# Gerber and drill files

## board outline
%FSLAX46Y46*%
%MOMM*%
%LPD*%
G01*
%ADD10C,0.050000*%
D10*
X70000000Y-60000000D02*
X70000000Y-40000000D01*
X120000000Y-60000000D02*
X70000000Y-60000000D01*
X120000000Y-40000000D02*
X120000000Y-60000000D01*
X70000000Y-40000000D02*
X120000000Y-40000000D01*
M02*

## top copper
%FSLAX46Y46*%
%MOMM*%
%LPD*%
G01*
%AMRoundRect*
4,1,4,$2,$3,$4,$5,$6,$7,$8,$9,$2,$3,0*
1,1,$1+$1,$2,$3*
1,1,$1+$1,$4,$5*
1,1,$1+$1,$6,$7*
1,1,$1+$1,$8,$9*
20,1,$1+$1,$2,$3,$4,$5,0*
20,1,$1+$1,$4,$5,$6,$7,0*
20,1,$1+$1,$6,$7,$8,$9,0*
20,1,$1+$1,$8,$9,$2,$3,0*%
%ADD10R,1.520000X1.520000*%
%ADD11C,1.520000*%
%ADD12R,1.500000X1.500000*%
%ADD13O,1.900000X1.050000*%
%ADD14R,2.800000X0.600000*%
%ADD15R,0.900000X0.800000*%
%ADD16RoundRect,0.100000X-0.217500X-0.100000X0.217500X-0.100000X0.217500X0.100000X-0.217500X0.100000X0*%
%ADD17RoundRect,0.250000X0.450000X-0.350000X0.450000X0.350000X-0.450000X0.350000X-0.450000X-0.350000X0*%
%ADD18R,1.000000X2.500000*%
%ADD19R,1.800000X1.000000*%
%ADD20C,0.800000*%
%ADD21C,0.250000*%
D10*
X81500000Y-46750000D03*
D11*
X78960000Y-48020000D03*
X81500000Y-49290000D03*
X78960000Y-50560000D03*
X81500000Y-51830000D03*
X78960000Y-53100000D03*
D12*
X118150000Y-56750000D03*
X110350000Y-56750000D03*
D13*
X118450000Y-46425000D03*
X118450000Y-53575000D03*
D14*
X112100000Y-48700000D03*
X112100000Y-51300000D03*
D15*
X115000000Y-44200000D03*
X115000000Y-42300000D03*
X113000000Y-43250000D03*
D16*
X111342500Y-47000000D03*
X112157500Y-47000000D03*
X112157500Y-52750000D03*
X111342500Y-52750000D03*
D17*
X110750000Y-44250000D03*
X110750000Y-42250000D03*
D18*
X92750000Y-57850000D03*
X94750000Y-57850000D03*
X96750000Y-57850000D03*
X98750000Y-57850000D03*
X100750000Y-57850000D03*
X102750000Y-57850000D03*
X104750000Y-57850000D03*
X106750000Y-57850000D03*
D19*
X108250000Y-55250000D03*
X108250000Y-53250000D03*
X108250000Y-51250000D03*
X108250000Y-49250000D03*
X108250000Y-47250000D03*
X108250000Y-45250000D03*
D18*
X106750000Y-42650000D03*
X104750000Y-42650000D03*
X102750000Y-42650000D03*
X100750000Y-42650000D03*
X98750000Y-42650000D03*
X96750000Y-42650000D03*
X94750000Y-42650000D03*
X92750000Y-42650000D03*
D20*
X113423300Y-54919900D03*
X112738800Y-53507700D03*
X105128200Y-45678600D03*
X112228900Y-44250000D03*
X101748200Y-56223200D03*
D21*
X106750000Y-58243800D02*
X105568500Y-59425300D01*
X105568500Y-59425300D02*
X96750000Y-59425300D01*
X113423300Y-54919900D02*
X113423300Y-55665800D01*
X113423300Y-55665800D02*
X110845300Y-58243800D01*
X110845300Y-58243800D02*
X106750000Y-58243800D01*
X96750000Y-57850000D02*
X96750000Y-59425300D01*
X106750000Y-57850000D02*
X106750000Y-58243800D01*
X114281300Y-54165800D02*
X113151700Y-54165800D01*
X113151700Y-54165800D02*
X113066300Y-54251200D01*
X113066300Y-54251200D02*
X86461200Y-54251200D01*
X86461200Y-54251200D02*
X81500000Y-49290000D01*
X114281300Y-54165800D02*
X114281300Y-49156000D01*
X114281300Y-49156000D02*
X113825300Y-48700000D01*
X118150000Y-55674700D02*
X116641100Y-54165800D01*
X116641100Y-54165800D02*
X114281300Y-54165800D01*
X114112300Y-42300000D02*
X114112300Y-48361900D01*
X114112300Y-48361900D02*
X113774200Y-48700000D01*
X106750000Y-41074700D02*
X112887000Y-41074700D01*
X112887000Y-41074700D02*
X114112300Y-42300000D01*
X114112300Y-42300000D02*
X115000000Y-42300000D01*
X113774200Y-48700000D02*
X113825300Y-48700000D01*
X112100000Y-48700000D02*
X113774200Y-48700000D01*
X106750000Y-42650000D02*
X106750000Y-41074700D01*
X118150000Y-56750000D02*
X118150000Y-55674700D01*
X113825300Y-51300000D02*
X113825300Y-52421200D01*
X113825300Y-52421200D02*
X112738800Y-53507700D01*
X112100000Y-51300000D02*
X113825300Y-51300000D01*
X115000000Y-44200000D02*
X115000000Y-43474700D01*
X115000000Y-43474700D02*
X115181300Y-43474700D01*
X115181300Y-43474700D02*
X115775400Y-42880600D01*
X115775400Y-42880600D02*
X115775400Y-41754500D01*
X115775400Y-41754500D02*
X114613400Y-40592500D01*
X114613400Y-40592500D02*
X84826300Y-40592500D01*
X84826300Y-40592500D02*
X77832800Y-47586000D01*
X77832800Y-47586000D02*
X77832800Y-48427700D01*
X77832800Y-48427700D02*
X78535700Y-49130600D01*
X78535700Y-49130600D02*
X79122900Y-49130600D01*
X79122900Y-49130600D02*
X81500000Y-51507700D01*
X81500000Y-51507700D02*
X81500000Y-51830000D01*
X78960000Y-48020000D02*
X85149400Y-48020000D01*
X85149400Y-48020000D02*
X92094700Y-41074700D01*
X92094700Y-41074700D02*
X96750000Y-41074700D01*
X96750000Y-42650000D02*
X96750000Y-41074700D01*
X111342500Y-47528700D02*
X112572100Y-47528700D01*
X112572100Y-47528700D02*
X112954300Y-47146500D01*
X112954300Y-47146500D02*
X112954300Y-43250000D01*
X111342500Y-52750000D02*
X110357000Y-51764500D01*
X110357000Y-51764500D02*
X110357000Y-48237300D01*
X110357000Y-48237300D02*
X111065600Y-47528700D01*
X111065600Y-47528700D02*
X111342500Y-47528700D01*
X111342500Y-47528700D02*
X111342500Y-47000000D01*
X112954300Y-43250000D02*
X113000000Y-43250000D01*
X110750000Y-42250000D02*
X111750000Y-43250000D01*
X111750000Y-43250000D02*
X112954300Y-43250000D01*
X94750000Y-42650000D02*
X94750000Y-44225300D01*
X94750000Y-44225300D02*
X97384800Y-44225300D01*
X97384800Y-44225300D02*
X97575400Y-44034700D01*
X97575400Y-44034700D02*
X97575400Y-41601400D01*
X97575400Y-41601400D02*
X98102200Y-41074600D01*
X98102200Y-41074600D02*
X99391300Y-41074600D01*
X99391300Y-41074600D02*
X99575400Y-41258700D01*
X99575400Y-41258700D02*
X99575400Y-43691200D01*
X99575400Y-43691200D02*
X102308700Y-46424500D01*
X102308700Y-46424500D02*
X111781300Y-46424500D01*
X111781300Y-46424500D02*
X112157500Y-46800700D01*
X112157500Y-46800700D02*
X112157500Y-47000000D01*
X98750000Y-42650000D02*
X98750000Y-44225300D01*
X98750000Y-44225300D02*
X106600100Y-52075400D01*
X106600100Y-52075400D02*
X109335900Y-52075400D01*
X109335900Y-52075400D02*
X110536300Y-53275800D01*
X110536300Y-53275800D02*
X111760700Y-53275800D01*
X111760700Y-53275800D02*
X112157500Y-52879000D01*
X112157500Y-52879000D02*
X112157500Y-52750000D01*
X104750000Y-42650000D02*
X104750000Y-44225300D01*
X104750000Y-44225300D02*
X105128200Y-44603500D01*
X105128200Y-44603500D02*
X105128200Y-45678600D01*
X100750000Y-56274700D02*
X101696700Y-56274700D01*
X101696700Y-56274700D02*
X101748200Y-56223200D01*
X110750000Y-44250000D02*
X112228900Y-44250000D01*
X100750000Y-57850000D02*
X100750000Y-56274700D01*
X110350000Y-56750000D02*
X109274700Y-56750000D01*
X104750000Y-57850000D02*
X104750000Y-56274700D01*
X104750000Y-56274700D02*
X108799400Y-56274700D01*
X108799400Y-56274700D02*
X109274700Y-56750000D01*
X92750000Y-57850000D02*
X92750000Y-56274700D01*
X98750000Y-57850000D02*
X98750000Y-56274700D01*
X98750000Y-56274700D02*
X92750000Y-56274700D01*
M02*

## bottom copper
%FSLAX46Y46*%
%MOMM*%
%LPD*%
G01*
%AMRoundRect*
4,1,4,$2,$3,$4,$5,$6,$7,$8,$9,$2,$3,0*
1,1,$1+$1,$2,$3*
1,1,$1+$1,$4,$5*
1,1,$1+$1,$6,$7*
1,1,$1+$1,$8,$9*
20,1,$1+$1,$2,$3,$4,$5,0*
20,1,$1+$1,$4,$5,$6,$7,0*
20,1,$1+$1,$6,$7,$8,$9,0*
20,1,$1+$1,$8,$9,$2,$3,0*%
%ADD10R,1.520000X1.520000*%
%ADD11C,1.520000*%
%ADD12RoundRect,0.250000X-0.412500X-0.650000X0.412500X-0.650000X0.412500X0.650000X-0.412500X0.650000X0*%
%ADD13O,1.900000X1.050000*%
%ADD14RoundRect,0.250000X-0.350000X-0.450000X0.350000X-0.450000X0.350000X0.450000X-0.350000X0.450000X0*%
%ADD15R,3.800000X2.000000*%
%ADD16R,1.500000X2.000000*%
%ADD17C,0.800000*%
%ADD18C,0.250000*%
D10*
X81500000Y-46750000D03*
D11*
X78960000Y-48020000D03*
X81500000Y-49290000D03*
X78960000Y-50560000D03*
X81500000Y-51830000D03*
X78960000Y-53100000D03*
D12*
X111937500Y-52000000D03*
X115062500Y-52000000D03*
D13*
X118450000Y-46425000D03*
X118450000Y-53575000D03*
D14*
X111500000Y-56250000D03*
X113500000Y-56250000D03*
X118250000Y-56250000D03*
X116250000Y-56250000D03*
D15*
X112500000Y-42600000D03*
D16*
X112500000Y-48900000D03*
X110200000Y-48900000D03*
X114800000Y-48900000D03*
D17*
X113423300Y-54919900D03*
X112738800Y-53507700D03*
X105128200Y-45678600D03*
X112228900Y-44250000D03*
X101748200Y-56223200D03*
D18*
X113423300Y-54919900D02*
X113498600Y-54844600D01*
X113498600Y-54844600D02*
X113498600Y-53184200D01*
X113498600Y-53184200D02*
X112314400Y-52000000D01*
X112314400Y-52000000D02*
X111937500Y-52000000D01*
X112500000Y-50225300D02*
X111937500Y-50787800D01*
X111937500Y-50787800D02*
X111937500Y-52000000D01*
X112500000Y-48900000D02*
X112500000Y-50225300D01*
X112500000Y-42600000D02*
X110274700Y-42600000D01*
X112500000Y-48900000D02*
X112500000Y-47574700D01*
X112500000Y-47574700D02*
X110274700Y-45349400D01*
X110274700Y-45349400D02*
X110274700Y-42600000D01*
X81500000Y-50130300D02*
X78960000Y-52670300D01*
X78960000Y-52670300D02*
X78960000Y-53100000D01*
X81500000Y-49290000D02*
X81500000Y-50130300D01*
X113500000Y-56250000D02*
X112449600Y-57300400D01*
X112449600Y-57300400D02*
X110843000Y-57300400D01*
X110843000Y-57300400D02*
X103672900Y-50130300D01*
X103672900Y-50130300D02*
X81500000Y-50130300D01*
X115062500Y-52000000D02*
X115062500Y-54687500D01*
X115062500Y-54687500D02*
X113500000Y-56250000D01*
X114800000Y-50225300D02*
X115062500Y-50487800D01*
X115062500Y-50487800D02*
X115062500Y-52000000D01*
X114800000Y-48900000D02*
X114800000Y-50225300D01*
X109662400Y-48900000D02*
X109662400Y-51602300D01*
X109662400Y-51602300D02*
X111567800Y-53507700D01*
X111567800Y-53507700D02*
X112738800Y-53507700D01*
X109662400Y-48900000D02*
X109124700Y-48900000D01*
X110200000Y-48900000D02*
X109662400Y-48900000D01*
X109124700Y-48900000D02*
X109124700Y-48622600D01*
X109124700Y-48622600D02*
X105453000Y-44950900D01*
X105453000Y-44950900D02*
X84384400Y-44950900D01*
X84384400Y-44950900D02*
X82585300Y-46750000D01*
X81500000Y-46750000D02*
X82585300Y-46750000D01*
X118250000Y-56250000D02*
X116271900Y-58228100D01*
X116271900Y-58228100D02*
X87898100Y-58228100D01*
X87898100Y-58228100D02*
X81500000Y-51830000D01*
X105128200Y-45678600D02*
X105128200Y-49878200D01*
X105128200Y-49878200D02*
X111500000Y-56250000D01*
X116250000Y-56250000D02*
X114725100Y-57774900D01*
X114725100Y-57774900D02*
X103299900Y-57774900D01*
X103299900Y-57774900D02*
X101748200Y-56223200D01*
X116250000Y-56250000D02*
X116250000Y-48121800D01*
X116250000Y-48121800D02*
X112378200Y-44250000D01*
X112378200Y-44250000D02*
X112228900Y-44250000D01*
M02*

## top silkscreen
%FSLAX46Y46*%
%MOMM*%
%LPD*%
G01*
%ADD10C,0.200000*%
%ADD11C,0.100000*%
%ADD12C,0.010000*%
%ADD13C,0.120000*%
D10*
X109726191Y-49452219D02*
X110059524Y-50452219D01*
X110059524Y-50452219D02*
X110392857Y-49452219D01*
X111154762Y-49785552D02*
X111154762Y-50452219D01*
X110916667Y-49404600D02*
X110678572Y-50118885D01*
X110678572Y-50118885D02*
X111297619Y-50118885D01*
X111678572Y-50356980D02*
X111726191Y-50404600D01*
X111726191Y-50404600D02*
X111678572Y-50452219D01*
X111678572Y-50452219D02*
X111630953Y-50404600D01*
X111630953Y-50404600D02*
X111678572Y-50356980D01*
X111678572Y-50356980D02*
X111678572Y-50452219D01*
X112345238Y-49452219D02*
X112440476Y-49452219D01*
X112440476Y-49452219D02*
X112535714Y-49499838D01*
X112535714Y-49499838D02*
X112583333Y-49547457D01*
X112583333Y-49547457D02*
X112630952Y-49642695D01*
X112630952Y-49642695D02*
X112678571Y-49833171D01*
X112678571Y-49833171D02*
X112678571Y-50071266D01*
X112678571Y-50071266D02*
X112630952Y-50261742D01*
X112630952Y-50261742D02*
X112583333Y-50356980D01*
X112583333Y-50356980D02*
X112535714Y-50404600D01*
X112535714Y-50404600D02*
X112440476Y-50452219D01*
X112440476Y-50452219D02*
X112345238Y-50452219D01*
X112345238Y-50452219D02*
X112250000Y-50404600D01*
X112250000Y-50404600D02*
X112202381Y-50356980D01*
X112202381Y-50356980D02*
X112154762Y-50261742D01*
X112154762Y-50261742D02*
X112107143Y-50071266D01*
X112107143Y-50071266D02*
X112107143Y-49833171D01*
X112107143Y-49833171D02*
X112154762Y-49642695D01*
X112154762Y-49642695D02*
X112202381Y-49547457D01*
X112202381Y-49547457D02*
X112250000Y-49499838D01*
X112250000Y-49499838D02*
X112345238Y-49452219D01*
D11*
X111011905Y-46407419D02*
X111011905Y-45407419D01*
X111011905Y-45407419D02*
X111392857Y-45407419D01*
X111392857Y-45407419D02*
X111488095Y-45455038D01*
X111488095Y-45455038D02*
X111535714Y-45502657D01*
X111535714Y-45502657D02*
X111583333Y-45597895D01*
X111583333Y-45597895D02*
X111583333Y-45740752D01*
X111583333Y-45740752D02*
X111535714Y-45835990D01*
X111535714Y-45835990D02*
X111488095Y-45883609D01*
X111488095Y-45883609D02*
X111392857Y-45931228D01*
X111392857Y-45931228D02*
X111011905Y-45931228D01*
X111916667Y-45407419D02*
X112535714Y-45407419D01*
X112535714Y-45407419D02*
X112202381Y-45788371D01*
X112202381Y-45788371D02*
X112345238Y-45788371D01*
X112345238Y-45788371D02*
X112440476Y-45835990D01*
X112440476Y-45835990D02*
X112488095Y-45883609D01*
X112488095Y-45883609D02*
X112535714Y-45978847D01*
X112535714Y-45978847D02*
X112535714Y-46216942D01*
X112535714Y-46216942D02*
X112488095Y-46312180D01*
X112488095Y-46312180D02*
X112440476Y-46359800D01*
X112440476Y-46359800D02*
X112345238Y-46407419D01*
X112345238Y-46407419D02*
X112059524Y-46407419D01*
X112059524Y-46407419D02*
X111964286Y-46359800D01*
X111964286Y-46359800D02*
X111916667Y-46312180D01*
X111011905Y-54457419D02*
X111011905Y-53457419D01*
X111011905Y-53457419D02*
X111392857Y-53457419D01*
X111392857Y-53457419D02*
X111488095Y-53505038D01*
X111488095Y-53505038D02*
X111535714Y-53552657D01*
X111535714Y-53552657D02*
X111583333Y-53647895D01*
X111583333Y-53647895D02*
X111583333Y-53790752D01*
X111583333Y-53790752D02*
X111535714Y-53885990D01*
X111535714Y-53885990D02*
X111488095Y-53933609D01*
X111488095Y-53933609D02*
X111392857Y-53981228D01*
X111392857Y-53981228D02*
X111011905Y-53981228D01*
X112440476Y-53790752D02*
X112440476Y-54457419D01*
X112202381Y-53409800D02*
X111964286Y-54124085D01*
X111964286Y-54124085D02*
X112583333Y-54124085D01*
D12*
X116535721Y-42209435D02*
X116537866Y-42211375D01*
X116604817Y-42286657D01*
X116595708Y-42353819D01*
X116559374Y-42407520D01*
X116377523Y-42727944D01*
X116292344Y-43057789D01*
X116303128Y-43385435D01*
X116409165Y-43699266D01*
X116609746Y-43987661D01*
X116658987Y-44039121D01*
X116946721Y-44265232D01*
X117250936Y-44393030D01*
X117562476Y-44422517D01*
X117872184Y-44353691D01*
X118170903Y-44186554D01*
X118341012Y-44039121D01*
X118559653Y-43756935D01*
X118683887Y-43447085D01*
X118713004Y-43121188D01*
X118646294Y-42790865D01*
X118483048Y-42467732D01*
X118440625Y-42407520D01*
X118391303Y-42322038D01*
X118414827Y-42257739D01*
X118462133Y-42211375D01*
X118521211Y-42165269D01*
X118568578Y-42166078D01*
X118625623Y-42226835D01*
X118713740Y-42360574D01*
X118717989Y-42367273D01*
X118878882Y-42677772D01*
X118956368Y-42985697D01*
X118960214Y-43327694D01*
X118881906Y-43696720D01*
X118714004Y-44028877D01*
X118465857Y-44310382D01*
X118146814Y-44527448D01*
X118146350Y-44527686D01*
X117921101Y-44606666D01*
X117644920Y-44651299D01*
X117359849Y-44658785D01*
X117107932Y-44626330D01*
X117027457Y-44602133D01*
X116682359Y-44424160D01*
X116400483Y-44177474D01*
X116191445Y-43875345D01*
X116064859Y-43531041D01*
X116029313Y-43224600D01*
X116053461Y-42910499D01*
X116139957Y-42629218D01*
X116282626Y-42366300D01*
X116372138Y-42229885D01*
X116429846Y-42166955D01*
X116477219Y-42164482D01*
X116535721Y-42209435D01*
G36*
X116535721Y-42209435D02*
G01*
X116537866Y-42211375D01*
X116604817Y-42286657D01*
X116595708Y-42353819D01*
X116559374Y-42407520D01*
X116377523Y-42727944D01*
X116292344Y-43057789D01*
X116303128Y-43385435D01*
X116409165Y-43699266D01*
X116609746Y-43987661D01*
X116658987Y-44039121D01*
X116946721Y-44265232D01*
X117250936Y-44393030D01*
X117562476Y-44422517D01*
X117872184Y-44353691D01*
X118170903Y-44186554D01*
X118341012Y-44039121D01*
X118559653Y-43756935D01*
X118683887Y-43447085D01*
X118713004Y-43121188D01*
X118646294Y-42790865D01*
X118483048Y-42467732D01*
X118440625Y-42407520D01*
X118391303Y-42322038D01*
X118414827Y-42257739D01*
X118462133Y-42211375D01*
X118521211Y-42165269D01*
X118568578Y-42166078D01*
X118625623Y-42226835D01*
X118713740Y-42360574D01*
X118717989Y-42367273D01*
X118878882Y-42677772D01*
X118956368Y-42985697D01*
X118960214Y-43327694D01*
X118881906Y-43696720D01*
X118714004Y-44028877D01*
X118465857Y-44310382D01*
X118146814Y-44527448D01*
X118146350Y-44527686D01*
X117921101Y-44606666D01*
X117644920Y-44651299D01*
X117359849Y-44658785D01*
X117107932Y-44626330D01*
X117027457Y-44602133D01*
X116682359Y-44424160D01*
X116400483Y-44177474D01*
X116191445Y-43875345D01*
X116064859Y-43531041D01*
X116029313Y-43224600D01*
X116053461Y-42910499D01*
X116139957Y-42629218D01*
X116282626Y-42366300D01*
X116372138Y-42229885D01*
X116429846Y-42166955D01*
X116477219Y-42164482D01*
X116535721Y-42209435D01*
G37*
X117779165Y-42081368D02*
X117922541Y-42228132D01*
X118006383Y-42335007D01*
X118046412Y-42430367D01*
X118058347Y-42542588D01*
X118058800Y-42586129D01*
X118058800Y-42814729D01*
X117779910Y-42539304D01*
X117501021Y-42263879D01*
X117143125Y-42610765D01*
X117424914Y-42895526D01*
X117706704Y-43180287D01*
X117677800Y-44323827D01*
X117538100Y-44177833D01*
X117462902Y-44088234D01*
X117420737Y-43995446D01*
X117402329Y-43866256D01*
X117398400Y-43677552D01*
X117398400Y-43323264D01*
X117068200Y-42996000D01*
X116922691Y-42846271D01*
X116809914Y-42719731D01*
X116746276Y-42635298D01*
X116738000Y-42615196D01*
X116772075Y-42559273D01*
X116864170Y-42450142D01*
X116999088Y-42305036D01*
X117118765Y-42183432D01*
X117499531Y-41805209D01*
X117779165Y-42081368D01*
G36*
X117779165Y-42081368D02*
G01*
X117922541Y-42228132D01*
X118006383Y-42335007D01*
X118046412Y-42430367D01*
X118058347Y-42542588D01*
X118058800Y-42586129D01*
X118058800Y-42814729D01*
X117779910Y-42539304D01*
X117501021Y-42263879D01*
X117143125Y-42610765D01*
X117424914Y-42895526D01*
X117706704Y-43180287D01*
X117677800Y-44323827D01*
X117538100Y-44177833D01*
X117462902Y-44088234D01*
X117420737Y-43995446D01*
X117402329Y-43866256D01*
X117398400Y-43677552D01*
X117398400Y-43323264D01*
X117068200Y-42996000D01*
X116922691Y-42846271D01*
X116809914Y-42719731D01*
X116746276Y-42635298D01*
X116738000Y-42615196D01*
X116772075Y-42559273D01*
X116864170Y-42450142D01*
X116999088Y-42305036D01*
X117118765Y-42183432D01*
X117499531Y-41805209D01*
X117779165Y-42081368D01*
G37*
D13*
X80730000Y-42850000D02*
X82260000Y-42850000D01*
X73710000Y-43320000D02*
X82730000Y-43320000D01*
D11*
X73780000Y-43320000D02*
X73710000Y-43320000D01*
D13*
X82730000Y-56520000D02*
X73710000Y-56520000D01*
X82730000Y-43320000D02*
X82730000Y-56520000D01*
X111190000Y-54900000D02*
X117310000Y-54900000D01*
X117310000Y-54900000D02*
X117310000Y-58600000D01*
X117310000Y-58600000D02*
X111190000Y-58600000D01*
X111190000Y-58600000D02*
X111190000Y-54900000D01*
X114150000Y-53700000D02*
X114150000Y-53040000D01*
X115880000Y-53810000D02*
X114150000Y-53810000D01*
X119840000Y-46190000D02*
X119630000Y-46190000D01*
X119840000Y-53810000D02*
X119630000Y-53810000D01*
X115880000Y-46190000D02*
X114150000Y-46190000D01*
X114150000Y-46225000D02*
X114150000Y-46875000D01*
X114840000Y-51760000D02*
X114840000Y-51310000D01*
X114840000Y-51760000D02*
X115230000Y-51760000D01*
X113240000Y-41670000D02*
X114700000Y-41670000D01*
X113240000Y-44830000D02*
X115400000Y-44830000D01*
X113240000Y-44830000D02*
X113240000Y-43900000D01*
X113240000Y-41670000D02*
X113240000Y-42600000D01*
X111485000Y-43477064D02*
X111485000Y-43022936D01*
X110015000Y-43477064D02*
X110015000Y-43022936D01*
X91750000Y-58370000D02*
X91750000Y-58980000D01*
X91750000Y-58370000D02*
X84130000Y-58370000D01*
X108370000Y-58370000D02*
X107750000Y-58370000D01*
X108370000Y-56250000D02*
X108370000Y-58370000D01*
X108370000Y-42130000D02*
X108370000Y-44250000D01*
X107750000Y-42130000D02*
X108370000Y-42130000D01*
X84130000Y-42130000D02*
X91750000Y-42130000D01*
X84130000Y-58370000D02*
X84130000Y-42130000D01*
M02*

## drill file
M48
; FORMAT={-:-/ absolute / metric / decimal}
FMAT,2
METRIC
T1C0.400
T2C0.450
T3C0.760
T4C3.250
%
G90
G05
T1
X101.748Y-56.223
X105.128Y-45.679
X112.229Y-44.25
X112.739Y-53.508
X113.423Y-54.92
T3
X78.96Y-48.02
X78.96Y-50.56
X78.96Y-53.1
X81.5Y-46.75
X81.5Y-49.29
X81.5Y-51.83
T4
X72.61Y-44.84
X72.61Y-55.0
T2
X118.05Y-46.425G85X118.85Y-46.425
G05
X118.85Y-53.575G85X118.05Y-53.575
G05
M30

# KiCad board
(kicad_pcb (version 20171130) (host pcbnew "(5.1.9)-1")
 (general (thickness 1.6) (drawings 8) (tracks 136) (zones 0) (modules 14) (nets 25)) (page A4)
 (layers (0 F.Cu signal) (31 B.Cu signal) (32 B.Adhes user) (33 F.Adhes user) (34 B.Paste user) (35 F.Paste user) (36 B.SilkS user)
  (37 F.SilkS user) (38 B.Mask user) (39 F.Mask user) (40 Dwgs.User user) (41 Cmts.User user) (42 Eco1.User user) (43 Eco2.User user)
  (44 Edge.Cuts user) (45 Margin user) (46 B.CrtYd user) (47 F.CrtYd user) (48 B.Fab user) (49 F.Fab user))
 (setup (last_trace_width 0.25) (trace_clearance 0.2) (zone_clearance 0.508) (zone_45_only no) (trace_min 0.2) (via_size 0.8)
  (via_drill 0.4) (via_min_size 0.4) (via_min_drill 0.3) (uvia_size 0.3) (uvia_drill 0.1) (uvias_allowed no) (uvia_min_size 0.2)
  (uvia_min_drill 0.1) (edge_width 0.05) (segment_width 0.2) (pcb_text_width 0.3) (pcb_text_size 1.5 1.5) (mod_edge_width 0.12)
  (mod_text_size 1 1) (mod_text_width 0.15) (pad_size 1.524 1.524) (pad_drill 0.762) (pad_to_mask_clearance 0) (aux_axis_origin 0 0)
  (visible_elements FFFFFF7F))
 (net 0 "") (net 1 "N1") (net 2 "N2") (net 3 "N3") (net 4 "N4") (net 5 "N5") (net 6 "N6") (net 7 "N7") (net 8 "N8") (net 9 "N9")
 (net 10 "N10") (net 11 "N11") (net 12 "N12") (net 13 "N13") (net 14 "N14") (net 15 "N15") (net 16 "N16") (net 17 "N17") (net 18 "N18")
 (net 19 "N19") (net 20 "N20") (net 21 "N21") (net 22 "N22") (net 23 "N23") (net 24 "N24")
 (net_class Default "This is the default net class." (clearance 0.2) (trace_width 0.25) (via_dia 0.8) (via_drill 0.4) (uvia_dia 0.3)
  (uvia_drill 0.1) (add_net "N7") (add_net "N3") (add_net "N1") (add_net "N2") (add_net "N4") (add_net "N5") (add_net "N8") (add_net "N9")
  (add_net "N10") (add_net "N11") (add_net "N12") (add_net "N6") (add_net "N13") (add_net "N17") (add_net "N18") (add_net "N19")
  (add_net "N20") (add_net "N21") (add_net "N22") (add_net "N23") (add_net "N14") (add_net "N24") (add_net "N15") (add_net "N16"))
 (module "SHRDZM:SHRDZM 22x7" (layer B.Cu) (at 96.25 49 180)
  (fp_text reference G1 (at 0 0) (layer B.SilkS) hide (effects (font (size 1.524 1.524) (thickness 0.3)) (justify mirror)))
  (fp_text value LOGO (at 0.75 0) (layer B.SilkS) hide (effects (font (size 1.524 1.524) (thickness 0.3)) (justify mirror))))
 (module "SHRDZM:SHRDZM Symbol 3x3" (layer F.Cu) (at 117.5 43.25)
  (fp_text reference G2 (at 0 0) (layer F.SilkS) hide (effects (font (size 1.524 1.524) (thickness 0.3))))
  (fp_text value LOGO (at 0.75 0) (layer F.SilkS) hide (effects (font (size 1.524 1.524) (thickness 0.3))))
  (fp_poly
   (pts (xy -0.964279 -1.040565) (xy -0.962134 -1.038625) (xy -0.895183 -0.963343) (xy -0.904292 -0.896181) (xy -0.940626 -0.84248)
    (xy -1.122477 -0.522056) (xy -1.207656 -0.192211) (xy -1.196872 0.135435) (xy -1.090835 0.449266) (xy -0.890254 0.737661)
    (xy -0.841013 0.789121) (xy -0.553279 1.015232) (xy -0.249064 1.14303) (xy 0.062476 1.172517) (xy 0.372184 1.103691)
    (xy 0.670903 0.936554) (xy 0.841012 0.789121) (xy 1.059653 0.506935) (xy 1.183887 0.197085) (xy 1.213004 -0.128812)
    (xy 1.146294 -0.459135) (xy 0.983048 -0.782268) (xy 0.940625 -0.84248) (xy 0.891303 -0.927962) (xy 0.914827 -0.992261)
    (xy 0.962133 -1.038625) (xy 1.021211 -1.084731) (xy 1.068578 -1.083922) (xy 1.125623 -1.023165) (xy 1.21374 -0.889426)
    (xy 1.217989 -0.882727) (xy 1.378882 -0.572228) (xy 1.456368 -0.264303) (xy 1.460214 0.077694) (xy 1.381906 0.44672)
    (xy 1.214004 0.778877) (xy 0.965857 1.060382) (xy 0.646814 1.277448) (xy 0.64635 1.277686) (xy 0.421101 1.356666) (xy 0.14492 1.401299)
    (xy -0.140151 1.408785) (xy -0.392068 1.37633) (xy -0.472543 1.352133) (xy -0.817641 1.17416) (xy -1.099517 0.927474)
    (xy -1.308555 0.625345) (xy -1.435141 0.281041) (xy -1.470687 -0.0254) (xy -1.446539 -0.339501) (xy -1.360043 -0.620782)
    (xy -1.217374 -0.8837) (xy -1.127862 -1.020115) (xy -1.070154 -1.083045) (xy -1.022781 -1.085518) (xy -0.964279 -1.040565))
   (layer F.SilkS) (width 0.01))
  (fp_poly
   (pts (xy 0.279165 -1.168632) (xy 0.422541 -1.021868) (xy 0.506383 -0.914993) (xy 0.546412 -0.819633) (xy 0.558347 -0.707412)
    (xy 0.5588 -0.663871) (xy 0.5588 -0.435271) (xy 0.27991 -0.710696) (xy 0.001021 -0.986121) (xy -0.356875 -0.639235)
    (xy -0.075086 -0.354474) (xy 0.206704 -0.069713) (xy 0.1778 1.073827) (xy 0.0381 0.927833) (xy -0.037098 0.838234)
    (xy -0.079263 0.745446) (xy -0.097671 0.616256) (xy -0.1016 0.427552) (xy -0.1016 0.073264) (xy -0.4318 -0.254) (xy -0.577309 -0.403729)
    (xy -0.690086 -0.530269) (xy -0.753724 -0.614702) (xy -0.762 -0.634804) (xy -0.727925 -0.690727) (xy -0.63583 -0.799858)
    (xy -0.500912 -0.944964) (xy -0.381235 -1.066568) (xy -0.000469 -1.444791) (xy 0.279165 -1.168632))
   (layer F.SilkS) (width 0.01)))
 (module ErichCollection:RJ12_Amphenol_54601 (layer F.Cu) (at 81.5 46.75 270)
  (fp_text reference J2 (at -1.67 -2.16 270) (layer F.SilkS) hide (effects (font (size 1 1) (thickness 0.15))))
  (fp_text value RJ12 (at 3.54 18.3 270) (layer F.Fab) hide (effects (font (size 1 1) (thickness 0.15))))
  (fp_line (start -3.9 0.77) (end -3.9 -0.76) (layer F.SilkS) (width 0.12))
  (fp_line (start -3.43 7.79) (end -3.43 -1.23) (layer F.SilkS) (width 0.12))
  (fp_line (start -3.43 7.72) (end -3.43 7.79) (layer F.SilkS) (width 0.1))
  (fp_line (start 9.77 -1.23) (end 9.77 7.79) (layer F.SilkS) (width 0.12))
  (fp_line (start -3.43 -1.23) (end 9.77 -1.23) (layer F.SilkS) (width 0.12))
  (pad 1 thru_hole rect (at 0 0 270) (size 1.52 1.52) (drill 0.76) (layers *.Cu *.Mask) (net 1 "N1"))
  (pad "" np_thru_hole circle (at -1.91 8.89 270) (size 3.25 3.25) (drill 3.25) (layers *.Cu *.Mask))
  (pad 2 thru_hole circle (at 1.27 2.54 270) (size 1.52 1.52) (drill 0.76) (layers *.Cu *.Mask) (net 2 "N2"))
  (pad 3 thru_hole circle (at 2.54 0 270) (size 1.52 1.52) (drill 0.76) (layers *.Cu *.Mask) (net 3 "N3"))
  (pad 4 thru_hole circle (at 3.81 2.54 270) (size 1.52 1.52) (drill 0.76) (layers *.Cu *.Mask) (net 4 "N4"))
  (pad 5 thru_hole circle (at 5.08 0 270) (size 1.52 1.52) (drill 0.76) (layers *.Cu *.Mask) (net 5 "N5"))
  (pad 6 thru_hole circle (at 6.35 2.54 270) (size 1.52 1.52) (drill 0.76) (layers *.Cu *.Mask) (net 3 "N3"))
  (pad "" np_thru_hole circle (at 8.25 8.89 270) (size 3.25 3.25) (drill 3.25) (layers *.Cu *.Mask)))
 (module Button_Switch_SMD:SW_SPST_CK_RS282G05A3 (layer F.Cu) (at 114.25 56.75)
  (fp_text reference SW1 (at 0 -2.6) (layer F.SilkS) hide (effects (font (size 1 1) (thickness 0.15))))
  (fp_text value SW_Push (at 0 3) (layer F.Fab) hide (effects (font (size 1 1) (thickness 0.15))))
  (fp_line (start -3.06 -1.85) (end 3.06 -1.85) (layer F.SilkS) (width 0.12))
  (fp_line (start 3.06 -1.85) (end 3.06 1.85) (layer F.SilkS) (width 0.12))
  (fp_line (start 3.06 1.85) (end -3.06 1.85) (layer F.SilkS) (width 0.12))
  (fp_line (start -3.06 1.85) (end -3.06 -1.85) (layer F.SilkS) (width 0.12))
  (pad 2 smd rect (at 3.9 0) (size 1.5 1.5) (layers F.Cu F.Paste F.Mask) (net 3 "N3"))
  (pad 1 smd rect (at -3.9 0) (size 1.5 1.5) (layers F.Cu F.Paste F.Mask) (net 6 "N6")))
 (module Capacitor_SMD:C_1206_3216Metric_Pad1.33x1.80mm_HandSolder (layer B.Cu) (at 113.5 52)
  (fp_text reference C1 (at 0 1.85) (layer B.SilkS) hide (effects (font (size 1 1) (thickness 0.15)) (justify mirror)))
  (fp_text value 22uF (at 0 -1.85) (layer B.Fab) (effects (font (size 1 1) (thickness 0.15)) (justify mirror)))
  (pad 1 smd roundrect (at -1.5625 0) (size 1.325 1.8) (layers B.Cu B.Paste B.Mask) (roundrect_rratio 0.188679) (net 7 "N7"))
  (pad 2 smd roundrect (at 1.5625 0) (size 1.325 1.8) (layers B.Cu B.Paste B.Mask) (roundrect_rratio 0.188679) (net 3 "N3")))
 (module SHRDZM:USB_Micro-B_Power (layer F.Cu) (at 117.25 50 90)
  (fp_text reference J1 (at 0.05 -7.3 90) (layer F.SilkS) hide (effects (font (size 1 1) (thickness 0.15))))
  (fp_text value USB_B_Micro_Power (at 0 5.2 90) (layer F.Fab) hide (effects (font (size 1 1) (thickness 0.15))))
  (fp_line (start -3.7 -3.1) (end -3.04 -3.1) (layer F.SilkS) (width 0.12))
  (fp_line (start -3.81 -1.37) (end -3.81 -3.1) (layer F.SilkS) (width 0.12))
  (fp_line (start 3.81 2.59) (end 3.81 2.38) (layer F.SilkS) (width 0.12))
  (fp_line (start -3.81 2.59) (end -3.81 2.38) (layer F.SilkS) (width 0.12))
  (fp_line (start 3.81 -1.37) (end 3.81 -3.1) (layer F.SilkS) (width 0.12))
  (fp_line (start 3.775 -3.1) (end 3.125 -3.1) (layer F.SilkS) (width 0.12))
  (fp_line (start -1.76 -2.41) (end -1.31 -2.41) (layer F.SilkS) (width 0.12))
  (fp_line (start -1.76 -2.41) (end -1.76 -2.02) (layer F.SilkS) (width 0.12))
  (pad "" thru_hole oval (at 3.575 1.2 90) (size 1.05 1.9) (drill oval 0.45 1.25) (layers *.Cu *.Mask))
  (pad "" thru_hole oval (at -3.575 1.2 270) (size 1.05 1.9) (drill oval 0.45 1.25) (layers *.Cu *.Mask))
  (pad 5 smd rect (at 1.3 -5.15 90) (size 0.6 2.8) (layers F.Cu F.Paste F.Mask) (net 3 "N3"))
  (pad 1 smd rect (at -1.3 -5.15 90) (size 0.6 2.8) (layers F.Cu F.Paste F.Mask) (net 1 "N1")))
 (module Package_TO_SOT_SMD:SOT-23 (layer F.Cu) (at 114 43.25 180)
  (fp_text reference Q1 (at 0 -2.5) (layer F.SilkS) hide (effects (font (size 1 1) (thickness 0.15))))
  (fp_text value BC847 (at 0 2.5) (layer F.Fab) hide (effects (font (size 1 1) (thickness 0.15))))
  (fp_line (start 0.76 1.58) (end -0.7 1.58) (layer F.SilkS) (width 0.12))
  (fp_line (start 0.76 -1.58) (end -1.4 -1.58) (layer F.SilkS) (width 0.12))
  (fp_line (start 0.76 -1.58) (end 0.76 -0.65) (layer F.SilkS) (width 0.12))
  (fp_line (start 0.76 1.58) (end 0.76 0.65) (layer F.SilkS) (width 0.12))
  (pad 1 smd rect (at -1 -0.95 180) (size 0.9 0.8) (layers F.Cu F.Paste F.Mask) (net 5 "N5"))
  (pad 2 smd rect (at -1 0.95 180) (size 0.9 0.8) (layers F.Cu F.Paste F.Mask) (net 3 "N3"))
  (pad 3 smd rect (at 1 0 180) (size 0.9 0.8) (layers F.Cu F.Paste F.Mask) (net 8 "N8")))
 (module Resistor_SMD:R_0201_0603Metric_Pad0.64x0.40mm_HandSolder (layer F.Cu) (at 111.75 47)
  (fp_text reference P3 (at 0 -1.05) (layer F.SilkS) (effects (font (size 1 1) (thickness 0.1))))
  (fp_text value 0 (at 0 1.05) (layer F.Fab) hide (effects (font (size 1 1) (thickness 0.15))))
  (pad "" smd roundrect (at -0.4325 0) (size 0.458 0.36) (layers F.Paste) (roundrect_rratio 0.25))
  (pad "" smd roundrect (at 0.4325 0) (size 0.458 0.36) (layers F.Paste) (roundrect_rratio 0.25))
  (pad 1 smd roundrect (at -0.4075 0) (size 0.635 0.4) (layers F.Cu F.Mask) (roundrect_rratio 0.25) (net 8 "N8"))
  (pad 2 smd roundrect (at 0.4075 0) (size 0.635 0.4) (layers F.Cu F.Mask) (roundrect_rratio 0.25) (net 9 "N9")))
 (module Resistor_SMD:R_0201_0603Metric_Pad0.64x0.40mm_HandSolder (layer F.Cu) (at 111.75 52.75)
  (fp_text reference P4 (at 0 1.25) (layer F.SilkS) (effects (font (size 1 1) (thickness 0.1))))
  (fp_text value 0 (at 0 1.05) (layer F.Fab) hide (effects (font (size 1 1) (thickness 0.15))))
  (pad 2 smd roundrect (at 0.4075 0) (size 0.635 0.4) (layers F.Cu F.Mask) (roundrect_rratio 0.25) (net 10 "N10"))
  (pad 1 smd roundrect (at -0.4075 0) (size 0.635 0.4) (layers F.Cu F.Mask) (roundrect_rratio 0.25) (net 8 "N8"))
  (pad "" smd roundrect (at 0.4325 0) (size 0.458 0.36) (layers F.Paste) (roundrect_rratio 0.25))
  (pad "" smd roundrect (at -0.4325 0) (size 0.458 0.36) (layers F.Paste) (roundrect_rratio 0.25)))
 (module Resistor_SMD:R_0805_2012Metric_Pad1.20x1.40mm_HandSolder (layer B.Cu) (at 112.5 56.25)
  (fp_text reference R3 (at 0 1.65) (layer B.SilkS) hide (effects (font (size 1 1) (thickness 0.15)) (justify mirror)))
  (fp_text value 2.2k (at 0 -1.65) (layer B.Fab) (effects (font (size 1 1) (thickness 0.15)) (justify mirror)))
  (pad 1 smd roundrect (at -1 0) (size 1.2 1.4) (layers B.Cu B.Paste B.Mask) (roundrect_rratio 0.208333) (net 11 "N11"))
  (pad 2 smd roundrect (at 1 0) (size 1.2 1.4) (layers B.Cu B.Paste B.Mask) (roundrect_rratio 0.208333) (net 3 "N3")))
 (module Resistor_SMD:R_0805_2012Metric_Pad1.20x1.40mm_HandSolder (layer F.Cu) (at 110.75 43.25 90)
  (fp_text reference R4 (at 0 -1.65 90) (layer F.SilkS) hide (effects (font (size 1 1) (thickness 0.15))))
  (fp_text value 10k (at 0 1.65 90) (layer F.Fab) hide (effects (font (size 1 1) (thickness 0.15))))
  (fp_line (start -0.227064 0.735) (end 0.227064 0.735) (layer F.SilkS) (width 0.12))
  (fp_line (start -0.227064 -0.735) (end 0.227064 -0.735) (layer F.SilkS) (width 0.12))
  (pad 1 smd roundrect (at -1 0 90) (size 1.2 1.4) (layers F.Cu F.Paste F.Mask) (roundrect_rratio 0.208333) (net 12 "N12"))
  (pad 2 smd roundrect (at 1 0 90) (size 1.2 1.4) (layers F.Cu F.Paste F.Mask) (roundrect_rratio 0.208333) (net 8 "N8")))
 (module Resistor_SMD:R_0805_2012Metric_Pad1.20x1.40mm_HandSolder (layer B.Cu) (at 117.25 56.25)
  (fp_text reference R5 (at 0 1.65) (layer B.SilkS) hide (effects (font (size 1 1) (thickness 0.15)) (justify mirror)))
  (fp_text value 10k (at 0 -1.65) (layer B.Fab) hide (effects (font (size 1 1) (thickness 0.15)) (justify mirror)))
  (pad 2 smd roundrect (at 1 0) (size 1.2 1.4) (layers B.Cu B.Paste B.Mask) (roundrect_rratio 0.208333) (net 5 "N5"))
  (pad 1 smd roundrect (at -1 0) (size 1.2 1.4) (layers B.Cu B.Paste B.Mask) (roundrect_rratio 0.208333) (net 12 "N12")))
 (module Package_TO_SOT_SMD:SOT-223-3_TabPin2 (layer B.Cu) (at 112.5 45.75 90)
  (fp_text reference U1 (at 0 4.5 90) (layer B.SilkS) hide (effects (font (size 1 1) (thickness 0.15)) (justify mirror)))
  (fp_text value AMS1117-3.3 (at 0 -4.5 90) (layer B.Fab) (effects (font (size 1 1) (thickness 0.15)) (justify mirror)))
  (pad 2 smd rect (at 3.15 0 90) (size 2 3.8) (layers B.Cu B.Paste B.Mask) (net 7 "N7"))
  (pad 2 smd rect (at -3.15 0 90) (size 2 1.5) (layers B.Cu B.Paste B.Mask) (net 7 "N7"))
  (pad 3 smd rect (at -3.15 -2.3 90) (size 2 1.5) (layers B.Cu B.Paste B.Mask) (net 1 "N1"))
  (pad 1 smd rect (at -3.15 2.3 90) (size 2 1.5) (layers B.Cu B.Paste B.Mask) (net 3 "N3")))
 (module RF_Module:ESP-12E (layer F.Cu) (at 96.25 50.25 90)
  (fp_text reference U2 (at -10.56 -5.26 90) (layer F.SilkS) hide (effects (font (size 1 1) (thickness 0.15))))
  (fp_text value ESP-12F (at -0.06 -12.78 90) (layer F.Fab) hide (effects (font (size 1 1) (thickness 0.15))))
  (fp_line (start -8.12 -4.5) (end -8.73 -4.5) (layer F.SilkS) (width 0.12))
  (fp_line (start -8.12 -4.5) (end -8.12 -12.12) (layer F.SilkS) (width 0.12))
  (fp_line (start -8.12 12.12) (end -8.12 11.5) (layer F.SilkS) (width 0.12))
  (fp_line (start -6 12.12) (end -8.12 12.12) (layer F.SilkS) (width 0.12))
  (fp_line (start 8.12 12.12) (end 6 12.12) (layer F.SilkS) (width 0.12))
  (fp_line (start 8.12 11.5) (end 8.12 12.12) (layer F.SilkS) (width 0.12))
  (fp_line (start 8.12 -12.12) (end 8.12 -4.5) (layer F.SilkS) (width 0.12))
  (fp_line (start -8.12 -12.12) (end 8.12 -12.12) (layer F.SilkS) (width 0.12))
  (pad 1 smd rect (at -7.6 -3.5 90) (size 2.5 1) (layers F.Cu F.Paste F.Mask) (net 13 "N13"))
  (pad 2 smd rect (at -7.6 -1.5 90) (size 2.5 1) (layers F.Cu F.Paste F.Mask) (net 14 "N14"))
  (pad 3 smd rect (at -7.6 0.5 90) (size 2.5 1) (layers F.Cu F.Paste F.Mask) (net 7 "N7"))
  (pad 4 smd rect (at -7.6 2.5 90) (size 2.5 1) (layers F.Cu F.Paste F.Mask) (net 13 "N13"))
  (pad 5 smd rect (at -7.6 4.5 90) (size 2.5 1) (layers F.Cu F.Paste F.Mask) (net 12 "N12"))
  (pad 6 smd rect (at -7.6 6.5 90) (size 2.5 1) (layers F.Cu F.Paste F.Mask) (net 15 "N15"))
  (pad 7 smd rect (at -7.6 8.5 90) (size 2.5 1) (layers F.Cu F.Paste F.Mask) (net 6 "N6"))
  (pad 8 smd rect (at -7.6 10.5 90) (size 2.5 1) (layers F.Cu F.Paste F.Mask) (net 7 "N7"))
  (pad 9 smd rect (at -5 12 90) (size 1 1.8) (layers F.Cu F.Paste F.Mask) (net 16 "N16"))
  (pad 10 smd rect (at -3 12 90) (size 1 1.8) (layers F.Cu F.Paste F.Mask) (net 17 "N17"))
  (pad 11 smd rect (at -1 12 90) (size 1 1.8) (layers F.Cu F.Paste F.Mask) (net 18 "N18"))
  (pad 12 smd rect (at 1 12 90) (size 1 1.8) (layers F.Cu F.Paste F.Mask) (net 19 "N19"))
  (pad 13 smd rect (at 3 12 90) (size 1 1.8) (layers F.Cu F.Paste F.Mask) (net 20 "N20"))
  (pad 14 smd rect (at 5 12 90) (size 1 1.8) (layers F.Cu F.Paste F.Mask) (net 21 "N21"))
  (pad 15 smd rect (at 7.6 10.5 90) (size 2.5 1) (layers F.Cu F.Paste F.Mask) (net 3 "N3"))
  (pad 16 smd rect (at 7.6 8.5 90) (size 2.5 1) (layers F.Cu F.Paste F.Mask) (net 11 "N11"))
  (pad 17 smd rect (at 7.6 6.5 90) (size 2.5 1) (layers F.Cu F.Paste F.Mask) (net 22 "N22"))
  (pad 18 smd rect (at 7.6 4.5 90) (size 2.5 1) (layers F.Cu F.Paste F.Mask) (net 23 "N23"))
  (pad 19 smd rect (at 7.6 2.5 90) (size 2.5 1) (layers F.Cu F.Paste F.Mask) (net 10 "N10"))
  (pad 20 smd rect (at 7.6 0.5 90) (size 2.5 1) (layers F.Cu F.Paste F.Mask) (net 2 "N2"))
  (pad 21 smd rect (at 7.6 -1.5 90) (size 2.5 1) (layers F.Cu F.Paste F.Mask) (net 9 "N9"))
  (pad 22 smd rect (at 7.6 -3.5 90) (size 2.5 1) (layers F.Cu F.Paste F.Mask) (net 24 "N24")))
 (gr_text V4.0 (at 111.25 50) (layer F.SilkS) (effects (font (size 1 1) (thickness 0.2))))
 (gr_line (start 70 60) (end 70 40) (layer Edge.Cuts) (width 0.05))
 (gr_line (start 120 60) (end 70 60) (layer Edge.Cuts) (width 0.05))
 (gr_line (start 120 40) (end 120 60) (layer Edge.Cuts) (width 0.05))
 (gr_line (start 70 40) (end 120 40) (layer Edge.Cuts) (width 0.05))
 (segment (start 106.75 58.2438) (end 105.5685 59.4253) (width 0.25) (layer F.Cu) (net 7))
 (segment (start 105.5685 59.4253) (end 96.75 59.4253) (width 0.25) (layer F.Cu) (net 7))
 (segment (start 113.4233 54.9199) (end 113.4233 55.6658) (width 0.25) (layer F.Cu) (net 7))
 (segment (start 113.4233 55.6658) (end 110.8453 58.2438) (width 0.25) (layer F.Cu) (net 7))
 (segment (start 110.8453 58.2438) (end 106.75 58.2438) (width 0.25) (layer F.Cu) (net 7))
 (segment (start 96.75 57.85) (end 96.75 59.4253) (width 0.25) (layer F.Cu) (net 7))
 (segment (start 113.4233 54.9199) (end 113.4986 54.8446) (width 0.25) (layer B.Cu) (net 7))
 (segment (start 113.4986 54.8446) (end 113.4986 53.1842) (width 0.25) (layer B.Cu) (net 7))
 (segment (start 113.4986 53.1842) (end 112.3144 52) (width 0.25) (layer B.Cu) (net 7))
 (segment (start 112.3144 52) (end 111.9375 52) (width 0.25) (layer B.Cu) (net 7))
 (segment (start 106.75 57.85) (end 106.75 58.2438) (width 0.25) (layer F.Cu) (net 7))
 (segment (start 112.5 50.2253) (end 111.9375 50.7878) (width 0.25) (layer B.Cu) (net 7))
 (segment (start 111.9375 50.7878) (end 111.9375 52) (width 0.25) (layer B.Cu) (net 7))
 (segment (start 112.5 48.9) (end 112.5 50.2253) (width 0.25) (layer B.Cu) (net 7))
 (segment (start 112.5 42.6) (end 110.2747 42.6) (width 0.25) (layer B.Cu) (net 7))
 (segment (start 112.5 48.9) (end 112.5 47.5747) (width 0.25) (layer B.Cu) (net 7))
 (segment (start 112.5 47.5747) (end 110.2747 45.3494) (width 0.25) (layer B.Cu) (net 7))
 (segment (start 110.2747 45.3494) (end 110.2747 42.6) (width 0.25) (layer B.Cu) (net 7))
 (via (at 113.4233 54.9199) (size 0.8) (layers F.Cu B.Cu) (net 7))
 (segment (start 114.2813 54.1658) (end 113.1517 54.1658) (width 0.25) (layer F.Cu) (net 3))
 (segment (start 113.1517 54.1658) (end 113.0663 54.2512) (width 0.25) (layer F.Cu) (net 3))
 (segment (start 113.0663 54.2512) (end 86.4612 54.2512) (width 0.25) (layer F.Cu) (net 3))
 (segment (start 86.4612 54.2512) (end 81.5 49.29) (width 0.25) (layer F.Cu) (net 3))
 (segment (start 114.2813 54.1658) (end 114.2813 49.156) (width 0.25) (layer F.Cu) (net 3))
 (segment (start 114.2813 49.156) (end 113.8253 48.7) (width 0.25) (layer F.Cu) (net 3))
 (segment (start 118.15 55.6747) (end 116.6411 54.1658) (width 0.25) (layer F.Cu) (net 3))
 (segment (start 116.6411 54.1658) (end 114.2813 54.1658) (width 0.25) (layer F.Cu) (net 3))
 (segment (start 81.5 50.1303) (end 78.96 52.6703) (width 0.25) (layer B.Cu) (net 3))
 (segment (start 78.96 52.6703) (end 78.96 53.1) (width 0.25) (layer B.Cu) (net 3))
 (segment (start 81.5 49.29) (end 81.5 50.1303) (width 0.25) (layer B.Cu) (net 3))
 (segment (start 113.5 56.25) (end 112.4496 57.3004) (width 0.25) (layer B.Cu) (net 3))
 (segment (start 112.4496 57.3004) (end 110.843 57.3004) (width 0.25) (layer B.Cu) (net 3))
 (segment (start 110.843 57.3004) (end 103.6729 50.1303) (width 0.25) (layer B.Cu) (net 3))
 (segment (start 103.6729 50.1303) (end 81.5 50.1303) (width 0.25) (layer B.Cu) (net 3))
 (segment (start 115.0625 52) (end 115.0625 54.6875) (width 0.25) (layer B.Cu) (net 3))
 (segment (start 115.0625 54.6875) (end 113.5 56.25) (width 0.25) (layer B.Cu) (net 3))
 (segment (start 114.1123 42.3) (end 114.1123 48.3619) (width 0.25) (layer F.Cu) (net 3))
 (segment (start 114.1123 48.3619) (end 113.7742 48.7) (width 0.25) (layer F.Cu) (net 3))
 (segment (start 106.75 41.0747) (end 112.887 41.0747) (width 0.25) (layer F.Cu) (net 3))
 (segment (start 112.887 41.0747) (end 114.1123 42.3) (width 0.25) (layer F.Cu) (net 3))
 (segment (start 114.1123 42.3) (end 115 42.3) (width 0.25) (layer F.Cu) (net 3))
 (segment (start 113.7742 48.7) (end 113.8253 48.7) (width 0.25) (layer F.Cu) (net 3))
 (segment (start 112.1 48.7) (end 113.7742 48.7) (width 0.25) (layer F.Cu) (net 3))
 (segment (start 106.75 42.65) (end 106.75 41.0747) (width 0.25) (layer F.Cu) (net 3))
 (segment (start 114.8 50.2253) (end 115.0625 50.4878) (width 0.25) (layer B.Cu) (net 3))
 (segment (start 115.0625 50.4878) (end 115.0625 52) (width 0.25) (layer B.Cu) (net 3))
 (segment (start 118.15 56.75) (end 118.15 55.6747) (width 0.25) (layer F.Cu) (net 3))
 (segment (start 114.8 48.9) (end 114.8 50.2253) (width 0.25) (layer B.Cu) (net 3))
 (segment (start 113.8253 51.3) (end 113.8253 52.4212) (width 0.25) (layer F.Cu) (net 1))
 (segment (start 113.8253 52.4212) (end 112.7388 53.5077) (width 0.25) (layer F.Cu) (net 1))
 (segment (start 109.6624 48.9) (end 109.6624 51.6023) (width 0.25) (layer B.Cu) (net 1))
 (segment (start 109.6624 51.6023) (end 111.5678 53.5077) (width 0.25) (layer B.Cu) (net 1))
 (segment (start 111.5678 53.5077) (end 112.7388 53.5077) (width 0.25) (layer B.Cu) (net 1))
 (segment (start 112.1 51.3) (end 113.8253 51.3) (width 0.25) (layer F.Cu) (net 1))
 (segment (start 109.6624 48.9) (end 109.1247 48.9) (width 0.25) (layer B.Cu) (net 1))
 (segment (start 110.2 48.9) (end 109.6624 48.9) (width 0.25) (layer B.Cu) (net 1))
 (segment (start 109.1247 48.9) (end 109.1247 48.6226) (width 0.25) (layer B.Cu) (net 1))
 (segment (start 109.1247 48.6226) (end 105.453 44.9509) (width 0.25) (layer B.Cu) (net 1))
 (segment (start 105.453 44.9509) (end 84.3844 44.9509) (width 0.25) (layer B.Cu) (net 1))
 (segment (start 84.3844 44.9509) (end 82.5853 46.75) (width 0.25) (layer B.Cu) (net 1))
 (segment (start 81.5 46.75) (end 82.5853 46.75) (width 0.25) (layer B.Cu) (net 1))
 (via (at 112.7388 53.5077) (size 0.8) (layers F.Cu B.Cu) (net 1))
 (segment (start 118.25 56.25) (end 116.2719 58.2281) (width 0.25) (layer B.Cu) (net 5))
 (segment (start 116.2719 58.2281) (end 87.8981 58.2281) (width 0.25) (layer B.Cu) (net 5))
 (segment (start 87.8981 58.2281) (end 81.5 51.83) (width 0.25) (layer B.Cu) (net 5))
 (segment (start 115 44.2) (end 115 43.4747) (width 0.25) (layer F.Cu) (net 5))
 (segment (start 115 43.4747) (end 115.1813 43.4747) (width 0.25) (layer F.Cu) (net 5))
 (segment (start 115.1813 43.4747) (end 115.7754 42.8806) (width 0.25) (layer F.Cu) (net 5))
 (segment (start 115.7754 42.8806) (end 115.7754 41.7545) (width 0.25) (layer F.Cu) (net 5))
 (segment (start 115.7754 41.7545) (end 114.6134 40.5925) (width 0.25) (layer F.Cu) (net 5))
 (segment (start 114.6134 40.5925) (end 84.8263 40.5925) (width 0.25) (layer F.Cu) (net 5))
 (segment (start 84.8263 40.5925) (end 77.8328 47.586) (width 0.25) (layer F.Cu) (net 5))
 (segment (start 77.8328 47.586) (end 77.8328 48.4277) (width 0.25) (layer F.Cu) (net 5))
 (segment (start 77.8328 48.4277) (end 78.5357 49.1306) (width 0.25) (layer F.Cu) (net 5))
 (segment (start 78.5357 49.1306) (end 79.1229 49.1306) (width 0.25) (layer F.Cu) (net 5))
 (segment (start 79.1229 49.1306) (end 81.5 51.5077) (width 0.25) (layer F.Cu) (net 5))
 (segment (start 81.5 51.5077) (end 81.5 51.83) (width 0.25) (layer F.Cu) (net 5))
 (segment (start 78.96 48.02) (end 85.1494 48.02) (width 0.25) (layer F.Cu) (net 2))
 (segment (start 85.1494 48.02) (end 92.0947 41.0747) (width 0.25) (layer F.Cu) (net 2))
 (segment (start 92.0947 41.0747) (end 96.75 41.0747) (width 0.25) (layer F.Cu) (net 2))
 (segment (start 96.75 42.65) (end 96.75 41.0747) (width 0.25) (layer F.Cu) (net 2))
 (segment (start 111.3425 47.5287) (end 112.5721 47.5287) (width 0.25) (layer F.Cu) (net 8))
 (segment (start 112.5721 47.5287) (end 112.9543 47.1465) (width 0.25) (layer F.Cu) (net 8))
 (segment (start 112.9543 47.1465) (end 112.9543 43.25) (width 0.25) (layer F.Cu) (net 8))
 (segment (start 111.3425 52.75) (end 110.357 51.7645) (width 0.25) (layer F.Cu) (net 8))
 (segment (start 110.357 51.7645) (end 110.357 48.2373) (width 0.25) (layer F.Cu) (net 8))
 (segment (start 110.357 48.2373) (end 111.0656 47.5287) (width 0.25) (layer F.Cu) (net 8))
 (segment (start 111.0656 47.5287) (end 111.3425 47.5287) (width 0.25) (layer F.Cu) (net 8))
 (segment (start 111.3425 47.5287) (end 111.3425 47) (width 0.25) (layer F.Cu) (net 8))
 (segment (start 112.9543 43.25) (end 113 43.25) (width 0.25) (layer F.Cu) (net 8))
 (segment (start 110.75 42.25) (end 111.75 43.25) (width 0.25) (layer F.Cu) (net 8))
 (segment (start 111.75 43.25) (end 112.9543 43.25) (width 0.25) (layer F.Cu) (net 8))
 (segment (start 94.75 42.65) (end 94.75 44.2253) (width 0.25) (layer F.Cu) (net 9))
 (segment (start 94.75 44.2253) (end 97.3848 44.2253) (width 0.25) (layer F.Cu) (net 9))
 (segment (start 97.3848 44.2253) (end 97.5754 44.0347) (width 0.25) (layer F.Cu) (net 9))
 (segment (start 97.5754 44.0347) (end 97.5754 41.6014) (width 0.25) (layer F.Cu) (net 9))
 (segment (start 97.5754 41.6014) (end 98.1022 41.0746) (width 0.25) (layer F.Cu) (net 9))
 (segment (start 98.1022 41.0746) (end 99.3913 41.0746) (width 0.25) (layer F.Cu) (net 9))
 (segment (start 99.3913 41.0746) (end 99.5754 41.2587) (width 0.25) (layer F.Cu) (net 9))
 (segment (start 99.5754 41.2587) (end 99.5754 43.6912) (width 0.25) (layer F.Cu) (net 9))
 (segment (start 99.5754 43.6912) (end 102.3087 46.4245) (width 0.25) (layer F.Cu) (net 9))
 (segment (start 102.3087 46.4245) (end 111.7813 46.4245) (width 0.25) (layer F.Cu) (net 9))
 (segment (start 111.7813 46.4245) (end 112.1575 46.8007) (width 0.25) (layer F.Cu) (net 9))
 (segment (start 112.1575 46.8007) (end 112.1575 47) (width 0.25) (layer F.Cu) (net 9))
 (segment (start 98.75 42.65) (end 98.75 44.2253) (width 0.25) (layer F.Cu) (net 10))
 (segment (start 98.75 44.2253) (end 106.6001 52.0754) (width 0.25) (layer F.Cu) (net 10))
 (segment (start 106.6001 52.0754) (end 109.3359 52.0754) (width 0.25) (layer F.Cu) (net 10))
 (segment (start 109.3359 52.0754) (end 110.5363 53.2758) (width 0.25) (layer F.Cu) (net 10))
 (segment (start 110.5363 53.2758) (end 111.7607 53.2758) (width 0.25) (layer F.Cu) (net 10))
 (segment (start 111.7607 53.2758) (end 112.1575 52.879) (width 0.25) (layer F.Cu) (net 10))
 (segment (start 112.1575 52.879) (end 112.1575 52.75) (width 0.25) (layer F.Cu) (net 10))
 (segment (start 104.75 42.65) (end 104.75 44.2253) (width 0.25) (layer F.Cu) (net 11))
 (segment (start 105.1282 45.6786) (end 105.1282 49.8782) (width 0.25) (layer B.Cu) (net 11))
 (segment (start 105.1282 49.8782) (end 111.5 56.25) (width 0.25) (layer B.Cu) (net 11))
 (segment (start 104.75 44.2253) (end 105.1282 44.6035) (width 0.25) (layer F.Cu) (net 11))
 (segment (start 105.1282 44.6035) (end 105.1282 45.6786) (width 0.25) (layer F.Cu) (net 11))
 (via (at 105.1282 45.6786) (size 0.8) (layers F.Cu B.Cu) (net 11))
 (segment (start 100.75 56.2747) (end 101.6967 56.2747) (width 0.25) (layer F.Cu) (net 12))
 (segment (start 101.6967 56.2747) (end 101.7482 56.2232) (width 0.25) (layer F.Cu) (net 12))
 (segment (start 116.25 56.25) (end 114.7251 57.7749) (width 0.25) (layer B.Cu) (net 12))
 (segment (start 114.7251 57.7749) (end 103.2999 57.7749) (width 0.25) (layer B.Cu) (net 12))
 (segment (start 103.2999 57.7749) (end 101.7482 56.2232) (width 0.25) (layer B.Cu) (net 12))
 (segment (start 110.75 44.25) (end 112.2289 44.25) (width 0.25) (layer F.Cu) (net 12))
 (segment (start 116.25 56.25) (end 116.25 48.1218) (width 0.25) (layer B.Cu) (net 12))
 (segment (start 116.25 48.1218) (end 112.3782 44.25) (width 0.25) (layer B.Cu) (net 12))
 (segment (start 112.3782 44.25) (end 112.2289 44.25) (width 0.25) (layer B.Cu) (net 12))
 (segment (start 100.75 57.85) (end 100.75 56.2747) (width 0.25) (layer F.Cu) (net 12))
 (via (at 112.2289 44.25) (size 0.8) (layers F.Cu B.Cu) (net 12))
 (via (at 101.7482 56.2232) (size 0.8) (layers F.Cu B.Cu) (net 12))
 (segment (start 110.35 56.75) (end 109.2747 56.75) (width 0.25) (layer F.Cu) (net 6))
 (segment (start 104.75 57.85) (end 104.75 56.2747) (width 0.25) (layer F.Cu) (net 6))
 (segment (start 104.75 56.2747) (end 108.7994 56.2747) (width 0.25) (layer F.Cu) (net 6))
 (segment (start 108.7994 56.2747) (end 109.2747 56.75) (width 0.25) (layer F.Cu) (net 6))
 (segment (start 92.75 57.85) (end 92.75 56.2747) (width 0.25) (layer F.Cu) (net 13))
 (segment (start 98.75 57.85) (end 98.75 56.2747) (width 0.25) (layer F.Cu) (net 13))
 (segment (start 98.75 56.2747) (end 92.75 56.2747) (width 0.25) (layer F.Cu) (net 13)))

